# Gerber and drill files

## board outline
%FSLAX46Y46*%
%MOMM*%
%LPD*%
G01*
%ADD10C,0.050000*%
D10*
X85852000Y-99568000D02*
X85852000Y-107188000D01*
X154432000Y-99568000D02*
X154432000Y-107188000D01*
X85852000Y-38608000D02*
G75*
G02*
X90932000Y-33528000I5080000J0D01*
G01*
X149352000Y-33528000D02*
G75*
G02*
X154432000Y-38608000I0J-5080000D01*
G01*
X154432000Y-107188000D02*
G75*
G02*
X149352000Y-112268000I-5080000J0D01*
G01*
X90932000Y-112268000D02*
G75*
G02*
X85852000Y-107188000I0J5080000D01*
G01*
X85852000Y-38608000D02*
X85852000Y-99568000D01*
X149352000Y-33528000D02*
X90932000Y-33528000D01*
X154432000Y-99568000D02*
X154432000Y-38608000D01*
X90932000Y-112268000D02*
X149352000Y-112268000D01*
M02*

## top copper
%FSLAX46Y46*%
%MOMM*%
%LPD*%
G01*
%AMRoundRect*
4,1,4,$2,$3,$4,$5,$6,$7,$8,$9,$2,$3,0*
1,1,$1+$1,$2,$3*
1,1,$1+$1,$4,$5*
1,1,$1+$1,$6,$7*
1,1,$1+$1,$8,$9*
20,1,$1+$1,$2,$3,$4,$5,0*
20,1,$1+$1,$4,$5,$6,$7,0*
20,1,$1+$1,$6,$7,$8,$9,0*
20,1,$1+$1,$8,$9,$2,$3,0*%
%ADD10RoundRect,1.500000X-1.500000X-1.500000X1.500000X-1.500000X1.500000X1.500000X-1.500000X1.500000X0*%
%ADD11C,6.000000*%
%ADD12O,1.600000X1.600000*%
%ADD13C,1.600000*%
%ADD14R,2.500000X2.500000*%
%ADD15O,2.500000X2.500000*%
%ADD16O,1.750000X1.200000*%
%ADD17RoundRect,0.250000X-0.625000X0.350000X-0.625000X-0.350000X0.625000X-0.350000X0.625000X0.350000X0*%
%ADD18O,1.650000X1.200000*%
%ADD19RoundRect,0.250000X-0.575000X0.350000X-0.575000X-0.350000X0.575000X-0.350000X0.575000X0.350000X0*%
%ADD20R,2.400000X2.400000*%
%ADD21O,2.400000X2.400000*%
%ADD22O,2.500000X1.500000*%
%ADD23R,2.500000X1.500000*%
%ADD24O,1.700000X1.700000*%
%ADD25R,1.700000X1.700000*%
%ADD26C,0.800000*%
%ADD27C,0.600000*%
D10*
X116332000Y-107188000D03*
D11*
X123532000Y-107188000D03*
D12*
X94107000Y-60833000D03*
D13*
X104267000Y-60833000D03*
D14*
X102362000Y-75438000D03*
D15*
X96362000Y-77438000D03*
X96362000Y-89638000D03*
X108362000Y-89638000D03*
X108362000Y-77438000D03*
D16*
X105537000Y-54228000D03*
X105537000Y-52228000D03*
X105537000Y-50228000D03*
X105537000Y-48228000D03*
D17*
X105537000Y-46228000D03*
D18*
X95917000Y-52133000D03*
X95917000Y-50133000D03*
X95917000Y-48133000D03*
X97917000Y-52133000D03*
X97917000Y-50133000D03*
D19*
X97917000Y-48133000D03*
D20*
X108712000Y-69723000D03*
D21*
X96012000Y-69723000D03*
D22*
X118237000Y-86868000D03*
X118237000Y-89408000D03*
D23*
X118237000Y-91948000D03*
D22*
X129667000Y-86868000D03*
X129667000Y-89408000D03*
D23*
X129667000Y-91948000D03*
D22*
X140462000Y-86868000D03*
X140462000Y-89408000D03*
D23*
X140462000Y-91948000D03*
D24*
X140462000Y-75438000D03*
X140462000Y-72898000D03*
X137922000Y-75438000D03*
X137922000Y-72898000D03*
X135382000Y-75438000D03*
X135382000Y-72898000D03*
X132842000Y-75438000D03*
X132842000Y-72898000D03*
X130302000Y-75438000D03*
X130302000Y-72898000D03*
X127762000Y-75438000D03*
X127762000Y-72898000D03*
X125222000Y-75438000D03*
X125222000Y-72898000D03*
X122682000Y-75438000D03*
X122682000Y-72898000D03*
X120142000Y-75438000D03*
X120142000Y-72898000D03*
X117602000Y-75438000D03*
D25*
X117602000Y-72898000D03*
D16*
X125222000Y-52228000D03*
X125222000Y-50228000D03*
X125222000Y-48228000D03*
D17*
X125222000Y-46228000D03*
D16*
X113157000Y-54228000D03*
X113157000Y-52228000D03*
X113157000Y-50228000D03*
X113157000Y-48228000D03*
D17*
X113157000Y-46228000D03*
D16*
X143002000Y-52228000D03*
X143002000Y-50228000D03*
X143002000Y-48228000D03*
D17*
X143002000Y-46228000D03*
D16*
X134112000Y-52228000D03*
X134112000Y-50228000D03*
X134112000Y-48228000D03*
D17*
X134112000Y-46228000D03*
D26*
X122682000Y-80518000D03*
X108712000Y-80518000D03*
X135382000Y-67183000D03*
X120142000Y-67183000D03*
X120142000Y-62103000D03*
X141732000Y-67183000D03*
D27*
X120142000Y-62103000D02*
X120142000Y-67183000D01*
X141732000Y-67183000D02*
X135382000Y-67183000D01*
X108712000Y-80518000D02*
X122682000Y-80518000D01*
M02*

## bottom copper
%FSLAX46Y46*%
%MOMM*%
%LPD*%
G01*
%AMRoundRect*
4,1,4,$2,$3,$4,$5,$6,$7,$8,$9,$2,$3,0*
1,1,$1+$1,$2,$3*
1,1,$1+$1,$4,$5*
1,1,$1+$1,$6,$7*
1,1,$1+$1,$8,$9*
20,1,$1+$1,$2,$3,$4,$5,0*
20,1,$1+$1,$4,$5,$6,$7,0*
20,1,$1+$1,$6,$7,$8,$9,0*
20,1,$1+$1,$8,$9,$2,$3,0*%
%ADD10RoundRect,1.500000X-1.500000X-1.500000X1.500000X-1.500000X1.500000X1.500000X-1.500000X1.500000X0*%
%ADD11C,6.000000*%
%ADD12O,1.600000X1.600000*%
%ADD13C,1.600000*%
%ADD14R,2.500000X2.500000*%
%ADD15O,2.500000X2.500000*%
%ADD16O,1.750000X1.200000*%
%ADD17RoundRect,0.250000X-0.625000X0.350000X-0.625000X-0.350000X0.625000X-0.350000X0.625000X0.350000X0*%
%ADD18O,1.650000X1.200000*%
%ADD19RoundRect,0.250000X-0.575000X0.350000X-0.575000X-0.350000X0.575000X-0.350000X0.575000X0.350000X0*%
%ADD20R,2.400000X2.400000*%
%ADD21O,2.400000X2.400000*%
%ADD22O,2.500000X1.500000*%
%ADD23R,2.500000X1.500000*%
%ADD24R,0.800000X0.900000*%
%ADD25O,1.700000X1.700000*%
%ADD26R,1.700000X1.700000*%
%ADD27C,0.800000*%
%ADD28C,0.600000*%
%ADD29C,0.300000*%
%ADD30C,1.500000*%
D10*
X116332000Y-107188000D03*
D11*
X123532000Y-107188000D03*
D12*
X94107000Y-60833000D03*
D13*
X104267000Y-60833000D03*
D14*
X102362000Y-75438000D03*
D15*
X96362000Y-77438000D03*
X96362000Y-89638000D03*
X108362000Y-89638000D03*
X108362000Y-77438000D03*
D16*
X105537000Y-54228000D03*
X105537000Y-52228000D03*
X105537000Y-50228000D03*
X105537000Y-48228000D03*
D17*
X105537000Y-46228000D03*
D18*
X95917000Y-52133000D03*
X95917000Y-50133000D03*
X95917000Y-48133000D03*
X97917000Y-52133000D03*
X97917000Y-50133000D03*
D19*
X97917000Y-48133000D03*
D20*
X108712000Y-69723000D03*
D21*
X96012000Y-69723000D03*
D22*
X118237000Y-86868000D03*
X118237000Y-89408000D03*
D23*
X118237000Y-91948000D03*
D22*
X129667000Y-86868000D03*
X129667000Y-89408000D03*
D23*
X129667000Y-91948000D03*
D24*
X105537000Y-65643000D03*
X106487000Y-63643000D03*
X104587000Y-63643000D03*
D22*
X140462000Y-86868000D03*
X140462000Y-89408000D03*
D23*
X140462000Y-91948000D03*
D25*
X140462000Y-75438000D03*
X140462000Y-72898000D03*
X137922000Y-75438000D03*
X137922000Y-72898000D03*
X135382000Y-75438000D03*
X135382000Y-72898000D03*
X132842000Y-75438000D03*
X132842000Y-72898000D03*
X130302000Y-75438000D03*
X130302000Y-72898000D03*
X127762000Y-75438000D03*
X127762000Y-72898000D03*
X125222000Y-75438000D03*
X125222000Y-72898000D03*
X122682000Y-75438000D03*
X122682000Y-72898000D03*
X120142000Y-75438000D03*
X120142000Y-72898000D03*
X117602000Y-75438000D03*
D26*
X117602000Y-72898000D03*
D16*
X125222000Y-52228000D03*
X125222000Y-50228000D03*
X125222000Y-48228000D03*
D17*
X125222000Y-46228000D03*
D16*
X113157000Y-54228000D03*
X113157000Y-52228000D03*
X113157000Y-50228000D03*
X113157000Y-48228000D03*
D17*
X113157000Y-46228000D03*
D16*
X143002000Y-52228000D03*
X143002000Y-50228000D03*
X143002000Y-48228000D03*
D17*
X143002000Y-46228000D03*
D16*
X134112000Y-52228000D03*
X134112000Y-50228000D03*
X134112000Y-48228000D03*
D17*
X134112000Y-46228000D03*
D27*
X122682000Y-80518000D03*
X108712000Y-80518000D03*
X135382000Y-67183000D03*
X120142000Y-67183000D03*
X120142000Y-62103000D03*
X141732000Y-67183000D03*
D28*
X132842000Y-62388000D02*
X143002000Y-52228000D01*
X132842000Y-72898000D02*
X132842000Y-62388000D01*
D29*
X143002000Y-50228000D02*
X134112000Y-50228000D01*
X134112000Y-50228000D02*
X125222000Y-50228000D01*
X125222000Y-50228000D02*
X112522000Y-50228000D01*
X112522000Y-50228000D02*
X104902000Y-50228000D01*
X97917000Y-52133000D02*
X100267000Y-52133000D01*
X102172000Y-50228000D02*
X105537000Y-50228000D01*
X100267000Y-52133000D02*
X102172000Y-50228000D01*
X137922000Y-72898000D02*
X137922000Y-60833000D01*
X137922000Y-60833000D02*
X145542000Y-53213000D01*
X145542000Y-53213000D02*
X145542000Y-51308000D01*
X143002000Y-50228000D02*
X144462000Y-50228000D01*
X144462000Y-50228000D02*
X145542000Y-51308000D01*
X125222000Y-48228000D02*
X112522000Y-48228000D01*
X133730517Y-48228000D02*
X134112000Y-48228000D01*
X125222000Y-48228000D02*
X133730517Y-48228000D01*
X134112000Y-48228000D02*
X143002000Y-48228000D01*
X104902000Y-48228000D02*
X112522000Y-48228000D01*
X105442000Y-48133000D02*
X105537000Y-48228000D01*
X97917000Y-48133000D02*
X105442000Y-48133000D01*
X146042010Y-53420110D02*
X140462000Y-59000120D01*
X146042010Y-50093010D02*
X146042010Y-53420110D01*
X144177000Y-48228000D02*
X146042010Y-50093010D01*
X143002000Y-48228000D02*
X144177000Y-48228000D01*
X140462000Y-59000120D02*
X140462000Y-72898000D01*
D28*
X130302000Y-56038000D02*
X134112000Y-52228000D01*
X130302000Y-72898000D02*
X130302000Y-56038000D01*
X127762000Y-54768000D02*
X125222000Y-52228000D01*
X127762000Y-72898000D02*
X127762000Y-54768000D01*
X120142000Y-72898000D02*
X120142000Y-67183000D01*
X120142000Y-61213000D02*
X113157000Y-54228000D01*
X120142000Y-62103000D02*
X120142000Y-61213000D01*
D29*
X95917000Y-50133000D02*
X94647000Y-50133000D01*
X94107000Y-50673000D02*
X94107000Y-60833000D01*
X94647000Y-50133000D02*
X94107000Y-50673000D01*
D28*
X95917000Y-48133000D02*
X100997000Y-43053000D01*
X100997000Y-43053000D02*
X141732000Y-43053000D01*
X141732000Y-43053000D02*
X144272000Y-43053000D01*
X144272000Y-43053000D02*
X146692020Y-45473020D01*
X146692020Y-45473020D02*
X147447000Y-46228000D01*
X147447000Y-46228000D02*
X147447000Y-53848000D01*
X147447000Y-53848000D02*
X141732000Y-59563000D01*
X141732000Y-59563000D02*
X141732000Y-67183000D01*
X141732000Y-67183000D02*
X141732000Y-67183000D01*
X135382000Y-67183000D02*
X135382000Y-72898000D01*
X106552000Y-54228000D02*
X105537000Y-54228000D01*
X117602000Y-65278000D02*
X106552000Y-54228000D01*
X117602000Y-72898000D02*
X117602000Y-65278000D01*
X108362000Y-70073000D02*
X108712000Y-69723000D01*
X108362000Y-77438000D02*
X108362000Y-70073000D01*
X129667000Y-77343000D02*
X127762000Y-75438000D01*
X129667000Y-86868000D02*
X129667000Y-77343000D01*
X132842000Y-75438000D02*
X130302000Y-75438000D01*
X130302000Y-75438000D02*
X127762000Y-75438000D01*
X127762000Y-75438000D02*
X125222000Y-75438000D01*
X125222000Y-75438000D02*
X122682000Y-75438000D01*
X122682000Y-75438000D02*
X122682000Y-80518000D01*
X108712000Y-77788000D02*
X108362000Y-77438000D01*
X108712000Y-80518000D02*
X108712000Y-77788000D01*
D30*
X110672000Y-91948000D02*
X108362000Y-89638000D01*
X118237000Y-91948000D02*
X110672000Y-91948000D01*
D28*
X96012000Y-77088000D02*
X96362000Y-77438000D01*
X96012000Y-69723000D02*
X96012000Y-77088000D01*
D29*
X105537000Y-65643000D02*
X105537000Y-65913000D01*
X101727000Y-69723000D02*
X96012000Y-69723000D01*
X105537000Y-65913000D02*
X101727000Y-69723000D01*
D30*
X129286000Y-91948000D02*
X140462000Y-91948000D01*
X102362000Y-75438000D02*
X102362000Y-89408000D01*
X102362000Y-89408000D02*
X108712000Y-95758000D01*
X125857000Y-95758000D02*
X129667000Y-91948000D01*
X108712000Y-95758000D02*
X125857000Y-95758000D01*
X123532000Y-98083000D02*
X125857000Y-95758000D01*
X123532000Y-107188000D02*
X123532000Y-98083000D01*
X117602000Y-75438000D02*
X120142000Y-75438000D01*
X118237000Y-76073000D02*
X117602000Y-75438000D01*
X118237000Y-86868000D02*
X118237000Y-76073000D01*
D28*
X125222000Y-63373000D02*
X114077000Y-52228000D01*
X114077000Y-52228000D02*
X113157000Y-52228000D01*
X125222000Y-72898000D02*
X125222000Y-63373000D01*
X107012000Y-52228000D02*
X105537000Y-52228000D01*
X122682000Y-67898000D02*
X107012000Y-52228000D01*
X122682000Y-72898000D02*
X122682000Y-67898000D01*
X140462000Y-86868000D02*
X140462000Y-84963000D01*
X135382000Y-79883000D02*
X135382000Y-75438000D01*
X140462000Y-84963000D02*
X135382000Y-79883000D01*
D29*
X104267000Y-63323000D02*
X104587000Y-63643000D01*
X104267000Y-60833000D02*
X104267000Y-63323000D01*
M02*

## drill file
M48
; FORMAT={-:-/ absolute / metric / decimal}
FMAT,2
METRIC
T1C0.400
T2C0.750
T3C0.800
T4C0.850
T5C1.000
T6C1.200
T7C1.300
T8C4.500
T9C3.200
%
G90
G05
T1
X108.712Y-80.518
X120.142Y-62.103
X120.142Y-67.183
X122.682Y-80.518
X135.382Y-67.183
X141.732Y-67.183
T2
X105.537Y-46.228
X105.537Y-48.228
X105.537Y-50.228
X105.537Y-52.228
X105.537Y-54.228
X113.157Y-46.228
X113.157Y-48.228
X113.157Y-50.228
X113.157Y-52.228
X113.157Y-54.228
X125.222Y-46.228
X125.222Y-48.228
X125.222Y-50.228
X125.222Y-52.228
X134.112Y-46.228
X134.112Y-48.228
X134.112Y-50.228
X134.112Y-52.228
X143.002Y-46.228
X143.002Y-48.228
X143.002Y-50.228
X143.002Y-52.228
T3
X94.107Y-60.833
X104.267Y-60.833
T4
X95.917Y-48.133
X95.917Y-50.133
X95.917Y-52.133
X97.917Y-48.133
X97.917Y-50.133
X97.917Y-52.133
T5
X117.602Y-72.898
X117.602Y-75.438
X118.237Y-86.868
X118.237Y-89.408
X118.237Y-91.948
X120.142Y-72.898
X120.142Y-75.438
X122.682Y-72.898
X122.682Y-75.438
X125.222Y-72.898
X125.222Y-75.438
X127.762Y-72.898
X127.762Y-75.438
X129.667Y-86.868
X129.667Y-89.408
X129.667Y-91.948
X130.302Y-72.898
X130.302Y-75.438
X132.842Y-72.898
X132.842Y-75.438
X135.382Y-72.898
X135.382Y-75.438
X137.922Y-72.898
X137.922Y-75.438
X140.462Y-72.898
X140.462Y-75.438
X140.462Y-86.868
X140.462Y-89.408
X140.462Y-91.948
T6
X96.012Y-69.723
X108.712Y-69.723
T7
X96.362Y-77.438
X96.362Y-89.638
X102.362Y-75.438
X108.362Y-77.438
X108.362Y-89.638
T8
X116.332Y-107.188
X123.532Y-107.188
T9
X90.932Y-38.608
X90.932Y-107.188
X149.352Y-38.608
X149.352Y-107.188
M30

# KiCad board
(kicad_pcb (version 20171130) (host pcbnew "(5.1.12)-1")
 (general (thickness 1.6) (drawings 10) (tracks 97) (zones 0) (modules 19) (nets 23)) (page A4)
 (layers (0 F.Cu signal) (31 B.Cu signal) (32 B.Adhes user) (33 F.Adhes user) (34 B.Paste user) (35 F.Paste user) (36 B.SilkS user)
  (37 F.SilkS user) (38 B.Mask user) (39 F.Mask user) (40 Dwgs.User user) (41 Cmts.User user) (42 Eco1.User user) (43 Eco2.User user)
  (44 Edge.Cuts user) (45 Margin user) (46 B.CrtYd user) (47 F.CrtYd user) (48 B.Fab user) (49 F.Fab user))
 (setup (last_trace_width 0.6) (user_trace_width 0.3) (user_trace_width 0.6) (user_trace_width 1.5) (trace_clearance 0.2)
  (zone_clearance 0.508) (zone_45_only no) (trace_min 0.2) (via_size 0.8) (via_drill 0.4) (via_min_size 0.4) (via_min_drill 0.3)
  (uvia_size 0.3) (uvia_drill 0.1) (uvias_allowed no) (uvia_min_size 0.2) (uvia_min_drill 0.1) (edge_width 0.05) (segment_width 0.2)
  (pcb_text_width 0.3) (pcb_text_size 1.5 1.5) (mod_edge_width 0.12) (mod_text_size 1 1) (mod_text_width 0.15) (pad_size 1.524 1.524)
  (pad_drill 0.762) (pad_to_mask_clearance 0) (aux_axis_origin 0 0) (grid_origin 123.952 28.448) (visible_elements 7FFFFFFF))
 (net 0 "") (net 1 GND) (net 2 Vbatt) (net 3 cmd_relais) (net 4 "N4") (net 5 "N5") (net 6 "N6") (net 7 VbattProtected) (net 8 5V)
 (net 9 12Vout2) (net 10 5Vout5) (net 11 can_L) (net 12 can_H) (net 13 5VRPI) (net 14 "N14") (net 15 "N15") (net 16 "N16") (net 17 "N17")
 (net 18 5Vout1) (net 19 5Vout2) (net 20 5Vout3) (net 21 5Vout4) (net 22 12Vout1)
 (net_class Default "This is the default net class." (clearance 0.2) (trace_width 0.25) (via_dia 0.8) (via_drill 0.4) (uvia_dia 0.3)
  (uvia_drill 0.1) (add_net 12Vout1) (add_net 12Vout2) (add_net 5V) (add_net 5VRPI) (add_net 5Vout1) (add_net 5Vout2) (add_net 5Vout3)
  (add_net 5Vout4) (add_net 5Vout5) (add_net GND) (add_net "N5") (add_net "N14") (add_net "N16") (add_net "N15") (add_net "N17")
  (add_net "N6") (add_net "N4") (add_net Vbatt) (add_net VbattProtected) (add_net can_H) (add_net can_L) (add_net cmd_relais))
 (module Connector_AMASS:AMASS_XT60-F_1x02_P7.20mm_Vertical (layer F.Cu) (at 116.332 107.188)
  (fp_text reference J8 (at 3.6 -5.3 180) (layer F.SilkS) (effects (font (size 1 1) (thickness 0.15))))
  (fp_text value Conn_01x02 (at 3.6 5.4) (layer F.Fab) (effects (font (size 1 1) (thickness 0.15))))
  (pad 1 thru_hole roundrect (at 0 0) (size 6 6) (drill 4.5) (layers *.Cu *.Mask) (roundrect_rratio 0.25) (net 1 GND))
  (pad 2 thru_hole circle (at 7.2 0) (size 6 6) (drill 4.5) (layers *.Cu *.Mask) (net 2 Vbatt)))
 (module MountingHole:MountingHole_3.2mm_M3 (layer F.Cu) (at 90.932 107.188)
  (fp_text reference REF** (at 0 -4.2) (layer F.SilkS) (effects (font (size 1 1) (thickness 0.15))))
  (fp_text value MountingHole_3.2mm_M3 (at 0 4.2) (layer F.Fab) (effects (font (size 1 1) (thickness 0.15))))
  (pad 1 np_thru_hole circle (at 0 0) (size 3.2 3.2) (drill 3.2) (layers *.Cu *.Mask)))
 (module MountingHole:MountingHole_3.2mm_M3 (layer F.Cu) (at 149.352 107.188)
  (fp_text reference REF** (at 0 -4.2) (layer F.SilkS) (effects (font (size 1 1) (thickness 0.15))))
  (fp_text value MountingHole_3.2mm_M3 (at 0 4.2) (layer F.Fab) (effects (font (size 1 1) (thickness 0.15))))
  (pad 1 np_thru_hole circle (at 0 0) (size 3.2 3.2) (drill 3.2) (layers *.Cu *.Mask)))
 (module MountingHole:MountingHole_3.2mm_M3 (layer F.Cu) (at 90.932 38.608)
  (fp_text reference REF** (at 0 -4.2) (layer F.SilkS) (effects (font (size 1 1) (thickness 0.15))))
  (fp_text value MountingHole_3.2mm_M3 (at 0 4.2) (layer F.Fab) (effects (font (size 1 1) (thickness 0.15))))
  (pad 1 np_thru_hole circle (at 0 0) (size 3.2 3.2) (drill 3.2) (layers *.Cu *.Mask)))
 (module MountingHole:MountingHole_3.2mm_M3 (layer F.Cu) (at 149.352 38.608)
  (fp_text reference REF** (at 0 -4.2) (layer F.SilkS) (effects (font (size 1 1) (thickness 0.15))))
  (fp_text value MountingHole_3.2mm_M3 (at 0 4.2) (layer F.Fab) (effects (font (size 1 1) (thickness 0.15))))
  (pad 1 np_thru_hole circle (at 0 0) (size 3.2 3.2) (drill 3.2) (layers *.Cu *.Mask)))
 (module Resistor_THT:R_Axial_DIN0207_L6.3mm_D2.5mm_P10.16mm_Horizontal (layer F.Cu) (at 104.267 60.833 180)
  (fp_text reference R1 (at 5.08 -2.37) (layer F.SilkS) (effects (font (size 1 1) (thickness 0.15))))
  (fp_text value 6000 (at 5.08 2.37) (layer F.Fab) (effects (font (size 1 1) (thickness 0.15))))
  (pad 2 thru_hole oval (at 10.16 0 180) (size 1.6 1.6) (drill 0.8) (layers *.Cu *.Mask) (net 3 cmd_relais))
  (pad 1 thru_hole circle (at 0 0 180) (size 1.6 1.6) (drill 0.8) (layers *.Cu *.Mask) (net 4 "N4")))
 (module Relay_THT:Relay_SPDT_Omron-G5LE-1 (layer F.Cu) (at 102.362 75.438)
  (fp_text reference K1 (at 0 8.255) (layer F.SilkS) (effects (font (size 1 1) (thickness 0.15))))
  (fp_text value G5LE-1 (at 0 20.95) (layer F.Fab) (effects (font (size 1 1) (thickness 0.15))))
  (pad 1 thru_hole rect (at 0 0) (size 2.5 2.5) (drill 1.3) (layers *.Cu *.Mask) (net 2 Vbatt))
  (pad 2 thru_hole oval (at -6 2) (size 2.5 2.5) (drill 1.3) (layers *.Cu *.Mask) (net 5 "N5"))
  (pad 3 thru_hole oval (at -6 14.2) (size 2.5 2.5) (drill 1.3) (layers *.Cu *.Mask) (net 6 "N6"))
  (pad 4 thru_hole oval (at 6 14.2) (size 2.5 2.5) (drill 1.3) (layers *.Cu *.Mask) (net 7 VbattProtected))
  (pad 5 thru_hole oval (at 6 2) (size 2.5 2.5) (drill 1.3) (layers *.Cu *.Mask) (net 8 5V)))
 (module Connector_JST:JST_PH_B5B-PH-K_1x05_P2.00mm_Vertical (layer F.Cu) (at 105.537 46.228 270)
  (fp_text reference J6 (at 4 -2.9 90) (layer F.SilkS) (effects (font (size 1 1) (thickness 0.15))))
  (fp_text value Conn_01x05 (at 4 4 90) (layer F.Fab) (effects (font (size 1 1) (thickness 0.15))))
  (pad 5 thru_hole oval (at 8 0 270) (size 1.2 1.75) (drill 0.75) (layers *.Cu *.Mask) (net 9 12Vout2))
  (pad 4 thru_hole oval (at 6 0 270) (size 1.2 1.75) (drill 0.75) (layers *.Cu *.Mask) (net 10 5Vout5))
  (pad 3 thru_hole oval (at 4 0 270) (size 1.2 1.75) (drill 0.75) (layers *.Cu *.Mask) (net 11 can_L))
  (pad 2 thru_hole oval (at 2 0 270) (size 1.2 1.75) (drill 0.75) (layers *.Cu *.Mask) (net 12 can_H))
  (pad 1 thru_hole roundrect (at 0 0 270) (size 1.2 1.75) (drill 0.75) (layers *.Cu *.Mask) (roundrect_rratio 0.208333) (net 1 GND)))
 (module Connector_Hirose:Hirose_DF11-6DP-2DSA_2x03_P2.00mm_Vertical (layer F.Cu) (at 97.917 48.133 270)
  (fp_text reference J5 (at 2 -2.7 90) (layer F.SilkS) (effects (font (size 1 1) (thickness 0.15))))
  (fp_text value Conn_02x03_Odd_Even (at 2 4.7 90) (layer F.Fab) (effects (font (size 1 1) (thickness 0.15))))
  (pad 6 thru_hole oval (at 4 2 270) (size 1.2 1.65) (drill 0.85) (layers *.Cu *.Mask) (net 1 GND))
  (pad 4 thru_hole oval (at 2 2 270) (size 1.2 1.65) (drill 0.85) (layers *.Cu *.Mask) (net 3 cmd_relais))
  (pad 2 thru_hole oval (at 0 2 270) (size 1.2 1.65) (drill 0.85) (layers *.Cu *.Mask) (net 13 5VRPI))
  (pad 5 thru_hole oval (at 4 0 270) (size 1.2 1.65) (drill 0.85) (layers *.Cu *.Mask) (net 11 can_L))
  (pad 3 thru_hole oval (at 2 0 270) (size 1.2 1.65) (drill 0.85) (layers *.Cu *.Mask) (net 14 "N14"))
  (pad 1 thru_hole roundrect (at 0 0 270) (size 1.2 1.65) (drill 0.85) (layers *.Cu *.Mask) (roundrect_rratio 0.208333) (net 12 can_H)))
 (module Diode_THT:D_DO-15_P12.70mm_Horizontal (layer F.Cu) (at 108.712 69.723 180)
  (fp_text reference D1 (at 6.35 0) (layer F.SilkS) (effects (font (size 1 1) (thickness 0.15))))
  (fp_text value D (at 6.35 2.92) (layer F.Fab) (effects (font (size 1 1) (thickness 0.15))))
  (pad 1 thru_hole rect (at 0 0 180) (size 2.4 2.4) (drill 1.2) (layers *.Cu *.Mask) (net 8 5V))
  (pad 2 thru_hole oval (at 12.7 0 180) (size 2.4 2.4) (drill 1.2) (layers *.Cu *.Mask) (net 5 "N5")))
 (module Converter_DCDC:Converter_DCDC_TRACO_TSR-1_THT (layer F.Cu) (at 118.237 91.948 90)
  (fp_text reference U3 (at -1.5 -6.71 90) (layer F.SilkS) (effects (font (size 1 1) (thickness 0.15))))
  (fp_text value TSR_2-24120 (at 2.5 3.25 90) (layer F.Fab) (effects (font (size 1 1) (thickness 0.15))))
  (pad 3 thru_hole oval (at 5.08 0 90) (size 1.5 2.5) (drill 1) (layers *.Cu *.Mask) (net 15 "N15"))
  (pad 2 thru_hole oval (at 2.54 0 90) (size 1.5 2.5) (drill 1) (layers *.Cu *.Mask) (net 1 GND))
  (pad 1 thru_hole rect (at 0 0 90) (size 1.5 2.5) (drill 1) (layers *.Cu *.Mask) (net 7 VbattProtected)))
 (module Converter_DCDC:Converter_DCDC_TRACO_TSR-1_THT (layer F.Cu) (at 129.667 91.948 90)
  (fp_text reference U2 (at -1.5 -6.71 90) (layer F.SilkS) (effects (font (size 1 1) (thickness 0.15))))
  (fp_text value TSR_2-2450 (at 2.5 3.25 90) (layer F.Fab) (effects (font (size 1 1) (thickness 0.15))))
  (pad 3 thru_hole oval (at 5.08 0 90) (size 1.5 2.5) (drill 1) (layers *.Cu *.Mask) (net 8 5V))
  (pad 2 thru_hole oval (at 2.54 0 90) (size 1.5 2.5) (drill 1) (layers *.Cu *.Mask) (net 1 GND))
  (pad 1 thru_hole rect (at 0 0 90) (size 1.5 2.5) (drill 1) (layers *.Cu *.Mask) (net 2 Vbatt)))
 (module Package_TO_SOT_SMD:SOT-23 (layer B.Cu) (at 105.537 64.643 270)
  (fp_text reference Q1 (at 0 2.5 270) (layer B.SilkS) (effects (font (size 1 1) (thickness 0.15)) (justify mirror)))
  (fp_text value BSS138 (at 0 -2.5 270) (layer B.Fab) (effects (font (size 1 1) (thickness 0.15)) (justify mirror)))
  (pad 3 smd rect (at 1 0 270) (size 0.9 0.8) (layers B.Cu B.Paste B.Mask) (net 5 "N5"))
  (pad 2 smd rect (at -1 -0.95 270) (size 0.9 0.8) (layers B.Cu B.Paste B.Mask) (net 1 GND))
  (pad 1 smd rect (at -1 0.95 270) (size 0.9 0.8) (layers B.Cu B.Paste B.Mask) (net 4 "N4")))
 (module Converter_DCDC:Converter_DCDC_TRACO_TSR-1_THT (layer F.Cu) (at 140.462 91.948 90)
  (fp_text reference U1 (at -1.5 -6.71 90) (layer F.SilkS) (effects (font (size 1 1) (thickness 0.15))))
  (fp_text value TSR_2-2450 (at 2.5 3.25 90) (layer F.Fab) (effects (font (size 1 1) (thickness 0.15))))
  (pad 3 thru_hole oval (at 5.08 0 90) (size 1.5 2.5) (drill 1) (layers *.Cu *.Mask) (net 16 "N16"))
  (pad 2 thru_hole oval (at 2.54 0 90) (size 1.5 2.5) (drill 1) (layers *.Cu *.Mask) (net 1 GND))
  (pad 1 thru_hole rect (at 0 0 90) (size 1.5 2.5) (drill 1) (layers *.Cu *.Mask) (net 2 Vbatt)))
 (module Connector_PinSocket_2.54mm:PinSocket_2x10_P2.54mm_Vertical (layer F.Cu) (at 117.602 72.898 90)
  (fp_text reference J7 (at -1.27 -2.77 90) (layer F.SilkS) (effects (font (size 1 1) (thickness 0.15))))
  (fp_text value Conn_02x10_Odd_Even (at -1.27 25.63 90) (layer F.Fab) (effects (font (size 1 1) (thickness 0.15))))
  (pad 20 thru_hole oval (at -2.54 22.86 90) (size 1.7 1.7) (drill 1) (layers *.Cu *.Mask) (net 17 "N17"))
  (pad 19 thru_hole oval (at 0 22.86 90) (size 1.7 1.7) (drill 1) (layers *.Cu *.Mask) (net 12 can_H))
  (pad 18 thru_hole oval (at -2.54 20.32 90) (size 1.7 1.7) (drill 1) (layers *.Cu *.Mask) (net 1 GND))
  (pad 17 thru_hole oval (at 0 20.32 90) (size 1.7 1.7) (drill 1) (layers *.Cu *.Mask) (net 11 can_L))
  (pad 16 thru_hole oval (at -2.54 17.78 90) (size 1.7 1.7) (drill 1) (layers *.Cu *.Mask) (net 16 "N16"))
  (pad 15 thru_hole oval (at 0 17.78 90) (size 1.7 1.7) (drill 1) (layers *.Cu *.Mask) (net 13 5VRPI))
  (pad 14 thru_hole oval (at -2.54 15.24 90) (size 1.7 1.7) (drill 1) (layers *.Cu *.Mask) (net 8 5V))
  (pad 13 thru_hole oval (at 0 15.24 90) (size 1.7 1.7) (drill 1) (layers *.Cu *.Mask) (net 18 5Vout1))
  (pad 12 thru_hole oval (at -2.54 12.7 90) (size 1.7 1.7) (drill 1) (layers *.Cu *.Mask) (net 8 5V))
  (pad 11 thru_hole oval (at 0 12.7 90) (size 1.7 1.7) (drill 1) (layers *.Cu *.Mask) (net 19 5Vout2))
  (pad 10 thru_hole oval (at -2.54 10.16 90) (size 1.7 1.7) (drill 1) (layers *.Cu *.Mask) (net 8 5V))
  (pad 9 thru_hole oval (at 0 10.16 90) (size 1.7 1.7) (drill 1) (layers *.Cu *.Mask) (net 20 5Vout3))
  (pad 8 thru_hole oval (at -2.54 7.62 90) (size 1.7 1.7) (drill 1) (layers *.Cu *.Mask) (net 8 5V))
  (pad 7 thru_hole oval (at 0 7.62 90) (size 1.7 1.7) (drill 1) (layers *.Cu *.Mask) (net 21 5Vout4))
  (pad 6 thru_hole oval (at -2.54 5.08 90) (size 1.7 1.7) (drill 1) (layers *.Cu *.Mask) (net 8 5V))
  (pad 5 thru_hole oval (at 0 5.08 90) (size 1.7 1.7) (drill 1) (layers *.Cu *.Mask) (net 10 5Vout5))
  (pad 4 thru_hole oval (at -2.54 2.54 90) (size 1.7 1.7) (drill 1) (layers *.Cu *.Mask) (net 15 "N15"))
  (pad 3 thru_hole oval (at 0 2.54 90) (size 1.7 1.7) (drill 1) (layers *.Cu *.Mask) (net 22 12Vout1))
  (pad 2 thru_hole oval (at -2.54 0 90) (size 1.7 1.7) (drill 1) (layers *.Cu *.Mask) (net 15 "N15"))
  (pad 1 thru_hole rect (at 0 0 90) (size 1.7 1.7) (drill 1) (layers *.Cu *.Mask) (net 9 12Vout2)))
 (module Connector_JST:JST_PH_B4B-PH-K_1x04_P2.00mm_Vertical (layer F.Cu) (at 125.222 46.228 270)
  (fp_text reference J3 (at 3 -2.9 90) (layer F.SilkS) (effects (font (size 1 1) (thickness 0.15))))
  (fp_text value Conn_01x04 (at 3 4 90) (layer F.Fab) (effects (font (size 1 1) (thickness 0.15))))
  (pad 4 thru_hole oval (at 6 0 270) (size 1.2 1.75) (drill 0.75) (layers *.Cu *.Mask) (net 20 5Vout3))
  (pad 3 thru_hole oval (at 4 0 270) (size 1.2 1.75) (drill 0.75) (layers *.Cu *.Mask) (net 11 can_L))
  (pad 2 thru_hole oval (at 2 0 270) (size 1.2 1.75) (drill 0.75) (layers *.Cu *.Mask) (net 12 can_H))
  (pad 1 thru_hole roundrect (at 0 0 270) (size 1.2 1.75) (drill 0.75) (layers *.Cu *.Mask) (roundrect_rratio 0.208333) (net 1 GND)))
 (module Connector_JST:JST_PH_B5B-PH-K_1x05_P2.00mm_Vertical (layer F.Cu) (at 113.157 46.228 270)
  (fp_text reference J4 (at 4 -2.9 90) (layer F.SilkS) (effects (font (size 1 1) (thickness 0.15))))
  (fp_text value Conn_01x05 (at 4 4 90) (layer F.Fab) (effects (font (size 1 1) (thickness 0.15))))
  (pad 5 thru_hole oval (at 8 0 270) (size 1.2 1.75) (drill 0.75) (layers *.Cu *.Mask) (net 22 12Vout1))
  (pad 4 thru_hole oval (at 6 0 270) (size 1.2 1.75) (drill 0.75) (layers *.Cu *.Mask) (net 21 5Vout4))
  (pad 3 thru_hole oval (at 4 0 270) (size 1.2 1.75) (drill 0.75) (layers *.Cu *.Mask) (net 11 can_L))
  (pad 2 thru_hole oval (at 2 0 270) (size 1.2 1.75) (drill 0.75) (layers *.Cu *.Mask) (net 12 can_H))
  (pad 1 thru_hole roundrect (at 0 0 270) (size 1.2 1.75) (drill 0.75) (layers *.Cu *.Mask) (roundrect_rratio 0.208333) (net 1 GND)))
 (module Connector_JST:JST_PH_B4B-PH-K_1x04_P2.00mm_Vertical (layer F.Cu) (at 143.002 46.228 270)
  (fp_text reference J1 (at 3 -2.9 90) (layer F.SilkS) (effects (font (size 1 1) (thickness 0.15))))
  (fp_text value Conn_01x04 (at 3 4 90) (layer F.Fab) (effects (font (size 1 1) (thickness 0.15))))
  (pad 4 thru_hole oval (at 6 0 270) (size 1.2 1.75) (drill 0.75) (layers *.Cu *.Mask) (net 18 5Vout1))
  (pad 3 thru_hole oval (at 4 0 270) (size 1.2 1.75) (drill 0.75) (layers *.Cu *.Mask) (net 11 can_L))
  (pad 2 thru_hole oval (at 2 0 270) (size 1.2 1.75) (drill 0.75) (layers *.Cu *.Mask) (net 12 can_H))
  (pad 1 thru_hole roundrect (at 0 0 270) (size 1.2 1.75) (drill 0.75) (layers *.Cu *.Mask) (roundrect_rratio 0.208333) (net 1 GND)))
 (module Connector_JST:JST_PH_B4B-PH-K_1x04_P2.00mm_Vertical (layer F.Cu) (at 134.112 46.228 270)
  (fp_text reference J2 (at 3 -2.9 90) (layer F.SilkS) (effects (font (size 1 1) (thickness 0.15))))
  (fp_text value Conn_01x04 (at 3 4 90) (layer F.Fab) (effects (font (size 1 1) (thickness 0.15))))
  (pad 4 thru_hole oval (at 6 0 270) (size 1.2 1.75) (drill 0.75) (layers *.Cu *.Mask) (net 19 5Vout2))
  (pad 3 thru_hole oval (at 4 0 270) (size 1.2 1.75) (drill 0.75) (layers *.Cu *.Mask) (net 11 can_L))
  (pad 2 thru_hole oval (at 2 0 270) (size 1.2 1.75) (drill 0.75) (layers *.Cu *.Mask) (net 12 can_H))
  (pad 1 thru_hole roundrect (at 0 0 270) (size 1.2 1.75) (drill 0.75) (layers *.Cu *.Mask) (roundrect_rratio 0.208333) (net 1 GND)))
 (gr_line (start 85.852 99.568) (end 85.852 107.188) (layer Edge.Cuts) (width 0.05))
 (gr_line (start 154.432 99.568) (end 154.432 107.188) (layer Edge.Cuts) (width 0.05))
 (gr_arc (start 90.932 38.608) (end 90.932 33.528) (angle -90) (layer Edge.Cuts) (width 0.05))
 (gr_arc (start 149.352 38.608) (end 154.432 38.608) (angle -90) (layer Edge.Cuts) (width 0.05))
 (gr_arc (start 149.352 107.188) (end 149.352 112.268) (angle -90) (layer Edge.Cuts) (width 0.05))
 (gr_arc (start 90.932 107.188) (end 85.852 107.188) (angle -90) (layer Edge.Cuts) (width 0.05))
 (gr_line (start 85.852 38.608) (end 85.852 99.568) (layer Edge.Cuts) (width 0.05))
 (gr_line (start 149.352 33.528) (end 90.932 33.528) (layer Edge.Cuts) (width 0.05))
 (gr_line (start 154.432 99.568) (end 154.432 38.608) (layer Edge.Cuts) (width 0.05))
 (gr_line (start 90.932 112.268) (end 149.352 112.268) (layer Edge.Cuts) (width 0.05))
 (via (at 122.682 80.518) (size 0.8) (drill 0.4) (layers F.Cu B.Cu) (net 8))
 (via (at 108.712 80.518) (size 0.8) (drill 0.4) (layers F.Cu B.Cu) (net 8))
 (via (at 135.382 67.183) (size 0.8) (drill 0.4) (layers F.Cu B.Cu) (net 13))
 (via (at 120.142 67.183) (size 0.8) (drill 0.4) (layers F.Cu B.Cu) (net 22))
 (via (at 120.142 62.103) (size 0.8) (drill 0.4) (layers F.Cu B.Cu) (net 22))
 (segment (start 120.142 62.103) (end 120.142 67.183) (width 0.6) (layer F.Cu) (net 22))
 (segment (start 132.842 62.388) (end 143.002 52.228) (width 0.6) (layer B.Cu) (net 18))
 (segment (start 132.842 72.898) (end 132.842 62.388) (width 0.6) (layer B.Cu) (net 18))
 (segment (start 143.002 50.228) (end 134.112 50.228) (width 0.3) (layer B.Cu) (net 11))
 (segment (start 134.112 50.228) (end 125.222 50.228) (width 0.3) (layer B.Cu) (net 11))
 (segment (start 125.222 50.228) (end 112.522 50.228) (width 0.3) (layer B.Cu) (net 11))
 (segment (start 112.522 50.228) (end 104.902 50.228) (width 0.3) (layer B.Cu) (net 11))
 (segment (start 97.917 52.133) (end 100.267 52.133) (width 0.3) (layer B.Cu) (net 11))
 (segment (start 102.172 50.228) (end 105.537 50.228) (width 0.3) (layer B.Cu) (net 11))
 (segment (start 100.267 52.133) (end 102.172 50.228) (width 0.3) (layer B.Cu) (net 11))
 (segment (start 137.922 72.898) (end 137.922 60.833) (width 0.3) (layer B.Cu) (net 11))
 (segment (start 137.922 60.833) (end 145.542 53.213) (width 0.3) (layer B.Cu) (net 11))
 (segment (start 145.542 53.213) (end 145.542 51.308) (width 0.3) (layer B.Cu) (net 11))
 (segment (start 143.002 50.228) (end 144.462 50.228) (width 0.3) (layer B.Cu) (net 11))
 (segment (start 144.462 50.228) (end 145.542 51.308) (width 0.3) (layer B.Cu) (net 11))
 (segment (start 125.222 48.228) (end 112.522 48.228) (width 0.3) (layer B.Cu) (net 12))
 (segment (start 133.730517 48.228) (end 134.112 48.228) (width 0.3) (layer B.Cu) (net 12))
 (segment (start 125.222 48.228) (end 133.730517 48.228) (width 0.3) (layer B.Cu) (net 12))
 (segment (start 134.112 48.228) (end 143.002 48.228) (width 0.3) (layer B.Cu) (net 12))
 (segment (start 104.902 48.228) (end 112.522 48.228) (width 0.3) (layer B.Cu) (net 12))
 (segment (start 105.442 48.133) (end 105.537 48.228) (width 0.3) (layer B.Cu) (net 12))
 (segment (start 97.917 48.133) (end 105.442 48.133) (width 0.3) (layer B.Cu) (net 12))
 (segment (start 146.04201 53.42011) (end 140.462 59.00012) (width 0.3) (layer B.Cu) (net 12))
 (segment (start 146.04201 50.09301) (end 146.04201 53.42011) (width 0.3) (layer B.Cu) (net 12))
 (segment (start 144.177 48.228) (end 146.04201 50.09301) (width 0.3) (layer B.Cu) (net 12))
 (segment (start 143.002 48.228) (end 144.177 48.228) (width 0.3) (layer B.Cu) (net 12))
 (segment (start 140.462 59.00012) (end 140.462 72.898) (width 0.3) (layer B.Cu) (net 12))
 (segment (start 130.302 56.038) (end 134.112 52.228) (width 0.6) (layer B.Cu) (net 19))
 (segment (start 130.302 72.898) (end 130.302 56.038) (width 0.6) (layer B.Cu) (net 19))
 (segment (start 127.762 54.768) (end 125.222 52.228) (width 0.6) (layer B.Cu) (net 20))
 (segment (start 127.762 72.898) (end 127.762 54.768) (width 0.6) (layer B.Cu) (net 20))
 (segment (start 120.142 72.898) (end 120.142 67.183) (width 0.6) (layer B.Cu) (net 22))
 (segment (start 120.142 61.213) (end 113.157 54.228) (width 0.6) (layer B.Cu) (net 22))
 (segment (start 120.142 62.103) (end 120.142 61.213) (width 0.6) (layer B.Cu) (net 22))
 (segment (start 95.917 50.133) (end 94.647 50.133) (width 0.3) (layer B.Cu) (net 3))
 (segment (start 94.107 50.673) (end 94.107 60.833) (width 0.3) (layer B.Cu) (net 3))
 (segment (start 94.647 50.133) (end 94.107 50.673) (width 0.3) (layer B.Cu) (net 3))
 (segment (start 95.917 48.133) (end 100.997 43.053) (width 0.6) (layer B.Cu) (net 13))
 (segment (start 100.997 43.053) (end 141.732 43.053) (width 0.6) (layer B.Cu) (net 13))
 (segment (start 141.732 43.053) (end 144.272 43.053) (width 0.6) (layer B.Cu) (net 13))
 (segment (start 144.272 43.053) (end 146.69202 45.47302) (width 0.6) (layer B.Cu) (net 13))
 (segment (start 146.69202 45.47302) (end 147.447 46.228) (width 0.6) (layer B.Cu) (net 13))
 (segment (start 147.447 46.228) (end 147.447 53.848) (width 0.6) (layer B.Cu) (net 13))
 (segment (start 147.447 53.848) (end 141.732 59.563) (width 0.6) (layer B.Cu) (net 13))
 (segment (start 141.732 59.563) (end 141.732 67.183) (width 0.6) (layer B.Cu) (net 13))
 (segment (start 141.732 67.183) (end 141.732 67.183) (width 0.6) (layer B.Cu) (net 13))
 (via (at 141.732 67.183) (size 0.8) (drill 0.4) (layers F.Cu B.Cu) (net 13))
 (segment (start 135.382 67.183) (end 135.382 72.898) (width 0.6) (layer B.Cu) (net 13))
 (segment (start 141.732 67.183) (end 135.382 67.183) (width 0.6) (layer F.Cu) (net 13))
 (segment (start 106.552 54.228) (end 105.537 54.228) (width 0.6) (layer B.Cu) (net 9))
 (segment (start 117.602 65.278) (end 106.552 54.228) (width 0.6) (layer B.Cu) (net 9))
 (segment (start 117.602 72.898) (end 117.602 65.278) (width 0.6) (layer B.Cu) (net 9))
 (segment (start 108.362 70.073) (end 108.712 69.723) (width 0.6) (layer B.Cu) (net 8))
 (segment (start 108.362 77.438) (end 108.362 70.073) (width 0.6) (layer B.Cu) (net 8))
 (segment (start 129.667 77.343) (end 127.762 75.438) (width 0.6) (layer B.Cu) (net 8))
 (segment (start 129.667 86.868) (end 129.667 77.343) (width 0.6) (layer B.Cu) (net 8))
 (segment (start 132.842 75.438) (end 130.302 75.438) (width 0.6) (layer B.Cu) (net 8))
 (segment (start 130.302 75.438) (end 127.762 75.438) (width 0.6) (layer B.Cu) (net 8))
 (segment (start 127.762 75.438) (end 125.222 75.438) (width 0.6) (layer B.Cu) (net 8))
 (segment (start 125.222 75.438) (end 122.682 75.438) (width 0.6) (layer B.Cu) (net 8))
 (segment (start 108.712 80.518) (end 122.682 80.518) (width 0.6) (layer F.Cu) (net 8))
 (segment (start 122.682 75.438) (end 122.682 80.518) (width 0.6) (layer B.Cu) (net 8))
 (segment (start 108.712 77.788) (end 108.362 77.438) (width 0.6) (layer B.Cu) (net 8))
 (segment (start 108.712 80.518) (end 108.712 77.788) (width 0.6) (layer B.Cu) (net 8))
 (segment (start 110.672 91.948) (end 108.362 89.638) (width 1.5) (layer B.Cu) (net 7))
 (segment (start 118.237 91.948) (end 110.672 91.948) (width 1.5) (layer B.Cu) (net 7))
 (segment (start 96.012 77.088) (end 96.362 77.438) (width 0.6) (layer B.Cu) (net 5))
 (segment (start 96.012 69.723) (end 96.012 77.088) (width 0.6) (layer B.Cu) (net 5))
 (segment (start 105.537 65.643) (end 105.537 65.913) (width 0.3) (layer B.Cu) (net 5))
 (segment (start 101.727 69.723) (end 96.012 69.723) (width 0.3) (layer B.Cu) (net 5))
 (segment (start 105.537 65.913) (end 101.727 69.723) (width 0.3) (layer B.Cu) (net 5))
 (segment (start 129.286 91.948) (end 140.462 91.948) (width 1.5) (layer B.Cu) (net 2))
 (segment (start 102.362 75.438) (end 102.362 89.408) (width 1.5) (layer B.Cu) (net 2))
 (segment (start 102.362 89.408) (end 108.712 95.758) (width 1.5) (layer B.Cu) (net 2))
 (segment (start 125.857 95.758) (end 129.667 91.948) (width 1.5) (layer B.Cu) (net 2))
 (segment (start 108.712 95.758) (end 125.857 95.758) (width 1.5) (layer B.Cu) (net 2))
 (segment (start 123.532 98.083) (end 125.857 95.758) (width 1.5) (layer B.Cu) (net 2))
 (segment (start 123.532 107.188) (end 123.532 98.083) (width 1.5) (layer B.Cu) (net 2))
 (segment (start 117.602 75.438) (end 120.142 75.438) (width 1.5) (layer B.Cu) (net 15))
 (segment (start 118.237 76.073) (end 117.602 75.438) (width 1.5) (layer B.Cu) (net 15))
 (segment (start 118.237 86.868) (end 118.237 76.073) (width 1.5) (layer B.Cu) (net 15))
 (segment (start 125.222 63.373) (end 114.077 52.228) (width 0.6) (layer B.Cu) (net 21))
 (segment (start 114.077 52.228) (end 113.157 52.228) (width 0.6) (layer B.Cu) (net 21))
 (segment (start 125.222 72.898) (end 125.222 63.373) (width 0.6) (layer B.Cu) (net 21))
 (segment (start 107.012 52.228) (end 105.537 52.228) (width 0.6) (layer B.Cu) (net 10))
 (segment (start 122.682 67.898) (end 107.012 52.228) (width 0.6) (layer B.Cu) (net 10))
 (segment (start 122.682 72.898) (end 122.682 67.898) (width 0.6) (layer B.Cu) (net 10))
 (segment (start 140.462 86.868) (end 140.462 84.963) (width 0.6) (layer B.Cu) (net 16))
 (segment (start 135.382 79.883) (end 135.382 75.438) (width 0.6) (layer B.Cu) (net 16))
 (segment (start 140.462 84.963) (end 135.382 79.883) (width 0.6) (layer B.Cu) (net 16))
 (segment (start 104.267 63.323) (end 104.587 63.643) (width 0.3) (layer B.Cu) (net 4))
 (segment (start 104.267 60.833) (end 104.267 63.323) (width 0.3) (layer B.Cu) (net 4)))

